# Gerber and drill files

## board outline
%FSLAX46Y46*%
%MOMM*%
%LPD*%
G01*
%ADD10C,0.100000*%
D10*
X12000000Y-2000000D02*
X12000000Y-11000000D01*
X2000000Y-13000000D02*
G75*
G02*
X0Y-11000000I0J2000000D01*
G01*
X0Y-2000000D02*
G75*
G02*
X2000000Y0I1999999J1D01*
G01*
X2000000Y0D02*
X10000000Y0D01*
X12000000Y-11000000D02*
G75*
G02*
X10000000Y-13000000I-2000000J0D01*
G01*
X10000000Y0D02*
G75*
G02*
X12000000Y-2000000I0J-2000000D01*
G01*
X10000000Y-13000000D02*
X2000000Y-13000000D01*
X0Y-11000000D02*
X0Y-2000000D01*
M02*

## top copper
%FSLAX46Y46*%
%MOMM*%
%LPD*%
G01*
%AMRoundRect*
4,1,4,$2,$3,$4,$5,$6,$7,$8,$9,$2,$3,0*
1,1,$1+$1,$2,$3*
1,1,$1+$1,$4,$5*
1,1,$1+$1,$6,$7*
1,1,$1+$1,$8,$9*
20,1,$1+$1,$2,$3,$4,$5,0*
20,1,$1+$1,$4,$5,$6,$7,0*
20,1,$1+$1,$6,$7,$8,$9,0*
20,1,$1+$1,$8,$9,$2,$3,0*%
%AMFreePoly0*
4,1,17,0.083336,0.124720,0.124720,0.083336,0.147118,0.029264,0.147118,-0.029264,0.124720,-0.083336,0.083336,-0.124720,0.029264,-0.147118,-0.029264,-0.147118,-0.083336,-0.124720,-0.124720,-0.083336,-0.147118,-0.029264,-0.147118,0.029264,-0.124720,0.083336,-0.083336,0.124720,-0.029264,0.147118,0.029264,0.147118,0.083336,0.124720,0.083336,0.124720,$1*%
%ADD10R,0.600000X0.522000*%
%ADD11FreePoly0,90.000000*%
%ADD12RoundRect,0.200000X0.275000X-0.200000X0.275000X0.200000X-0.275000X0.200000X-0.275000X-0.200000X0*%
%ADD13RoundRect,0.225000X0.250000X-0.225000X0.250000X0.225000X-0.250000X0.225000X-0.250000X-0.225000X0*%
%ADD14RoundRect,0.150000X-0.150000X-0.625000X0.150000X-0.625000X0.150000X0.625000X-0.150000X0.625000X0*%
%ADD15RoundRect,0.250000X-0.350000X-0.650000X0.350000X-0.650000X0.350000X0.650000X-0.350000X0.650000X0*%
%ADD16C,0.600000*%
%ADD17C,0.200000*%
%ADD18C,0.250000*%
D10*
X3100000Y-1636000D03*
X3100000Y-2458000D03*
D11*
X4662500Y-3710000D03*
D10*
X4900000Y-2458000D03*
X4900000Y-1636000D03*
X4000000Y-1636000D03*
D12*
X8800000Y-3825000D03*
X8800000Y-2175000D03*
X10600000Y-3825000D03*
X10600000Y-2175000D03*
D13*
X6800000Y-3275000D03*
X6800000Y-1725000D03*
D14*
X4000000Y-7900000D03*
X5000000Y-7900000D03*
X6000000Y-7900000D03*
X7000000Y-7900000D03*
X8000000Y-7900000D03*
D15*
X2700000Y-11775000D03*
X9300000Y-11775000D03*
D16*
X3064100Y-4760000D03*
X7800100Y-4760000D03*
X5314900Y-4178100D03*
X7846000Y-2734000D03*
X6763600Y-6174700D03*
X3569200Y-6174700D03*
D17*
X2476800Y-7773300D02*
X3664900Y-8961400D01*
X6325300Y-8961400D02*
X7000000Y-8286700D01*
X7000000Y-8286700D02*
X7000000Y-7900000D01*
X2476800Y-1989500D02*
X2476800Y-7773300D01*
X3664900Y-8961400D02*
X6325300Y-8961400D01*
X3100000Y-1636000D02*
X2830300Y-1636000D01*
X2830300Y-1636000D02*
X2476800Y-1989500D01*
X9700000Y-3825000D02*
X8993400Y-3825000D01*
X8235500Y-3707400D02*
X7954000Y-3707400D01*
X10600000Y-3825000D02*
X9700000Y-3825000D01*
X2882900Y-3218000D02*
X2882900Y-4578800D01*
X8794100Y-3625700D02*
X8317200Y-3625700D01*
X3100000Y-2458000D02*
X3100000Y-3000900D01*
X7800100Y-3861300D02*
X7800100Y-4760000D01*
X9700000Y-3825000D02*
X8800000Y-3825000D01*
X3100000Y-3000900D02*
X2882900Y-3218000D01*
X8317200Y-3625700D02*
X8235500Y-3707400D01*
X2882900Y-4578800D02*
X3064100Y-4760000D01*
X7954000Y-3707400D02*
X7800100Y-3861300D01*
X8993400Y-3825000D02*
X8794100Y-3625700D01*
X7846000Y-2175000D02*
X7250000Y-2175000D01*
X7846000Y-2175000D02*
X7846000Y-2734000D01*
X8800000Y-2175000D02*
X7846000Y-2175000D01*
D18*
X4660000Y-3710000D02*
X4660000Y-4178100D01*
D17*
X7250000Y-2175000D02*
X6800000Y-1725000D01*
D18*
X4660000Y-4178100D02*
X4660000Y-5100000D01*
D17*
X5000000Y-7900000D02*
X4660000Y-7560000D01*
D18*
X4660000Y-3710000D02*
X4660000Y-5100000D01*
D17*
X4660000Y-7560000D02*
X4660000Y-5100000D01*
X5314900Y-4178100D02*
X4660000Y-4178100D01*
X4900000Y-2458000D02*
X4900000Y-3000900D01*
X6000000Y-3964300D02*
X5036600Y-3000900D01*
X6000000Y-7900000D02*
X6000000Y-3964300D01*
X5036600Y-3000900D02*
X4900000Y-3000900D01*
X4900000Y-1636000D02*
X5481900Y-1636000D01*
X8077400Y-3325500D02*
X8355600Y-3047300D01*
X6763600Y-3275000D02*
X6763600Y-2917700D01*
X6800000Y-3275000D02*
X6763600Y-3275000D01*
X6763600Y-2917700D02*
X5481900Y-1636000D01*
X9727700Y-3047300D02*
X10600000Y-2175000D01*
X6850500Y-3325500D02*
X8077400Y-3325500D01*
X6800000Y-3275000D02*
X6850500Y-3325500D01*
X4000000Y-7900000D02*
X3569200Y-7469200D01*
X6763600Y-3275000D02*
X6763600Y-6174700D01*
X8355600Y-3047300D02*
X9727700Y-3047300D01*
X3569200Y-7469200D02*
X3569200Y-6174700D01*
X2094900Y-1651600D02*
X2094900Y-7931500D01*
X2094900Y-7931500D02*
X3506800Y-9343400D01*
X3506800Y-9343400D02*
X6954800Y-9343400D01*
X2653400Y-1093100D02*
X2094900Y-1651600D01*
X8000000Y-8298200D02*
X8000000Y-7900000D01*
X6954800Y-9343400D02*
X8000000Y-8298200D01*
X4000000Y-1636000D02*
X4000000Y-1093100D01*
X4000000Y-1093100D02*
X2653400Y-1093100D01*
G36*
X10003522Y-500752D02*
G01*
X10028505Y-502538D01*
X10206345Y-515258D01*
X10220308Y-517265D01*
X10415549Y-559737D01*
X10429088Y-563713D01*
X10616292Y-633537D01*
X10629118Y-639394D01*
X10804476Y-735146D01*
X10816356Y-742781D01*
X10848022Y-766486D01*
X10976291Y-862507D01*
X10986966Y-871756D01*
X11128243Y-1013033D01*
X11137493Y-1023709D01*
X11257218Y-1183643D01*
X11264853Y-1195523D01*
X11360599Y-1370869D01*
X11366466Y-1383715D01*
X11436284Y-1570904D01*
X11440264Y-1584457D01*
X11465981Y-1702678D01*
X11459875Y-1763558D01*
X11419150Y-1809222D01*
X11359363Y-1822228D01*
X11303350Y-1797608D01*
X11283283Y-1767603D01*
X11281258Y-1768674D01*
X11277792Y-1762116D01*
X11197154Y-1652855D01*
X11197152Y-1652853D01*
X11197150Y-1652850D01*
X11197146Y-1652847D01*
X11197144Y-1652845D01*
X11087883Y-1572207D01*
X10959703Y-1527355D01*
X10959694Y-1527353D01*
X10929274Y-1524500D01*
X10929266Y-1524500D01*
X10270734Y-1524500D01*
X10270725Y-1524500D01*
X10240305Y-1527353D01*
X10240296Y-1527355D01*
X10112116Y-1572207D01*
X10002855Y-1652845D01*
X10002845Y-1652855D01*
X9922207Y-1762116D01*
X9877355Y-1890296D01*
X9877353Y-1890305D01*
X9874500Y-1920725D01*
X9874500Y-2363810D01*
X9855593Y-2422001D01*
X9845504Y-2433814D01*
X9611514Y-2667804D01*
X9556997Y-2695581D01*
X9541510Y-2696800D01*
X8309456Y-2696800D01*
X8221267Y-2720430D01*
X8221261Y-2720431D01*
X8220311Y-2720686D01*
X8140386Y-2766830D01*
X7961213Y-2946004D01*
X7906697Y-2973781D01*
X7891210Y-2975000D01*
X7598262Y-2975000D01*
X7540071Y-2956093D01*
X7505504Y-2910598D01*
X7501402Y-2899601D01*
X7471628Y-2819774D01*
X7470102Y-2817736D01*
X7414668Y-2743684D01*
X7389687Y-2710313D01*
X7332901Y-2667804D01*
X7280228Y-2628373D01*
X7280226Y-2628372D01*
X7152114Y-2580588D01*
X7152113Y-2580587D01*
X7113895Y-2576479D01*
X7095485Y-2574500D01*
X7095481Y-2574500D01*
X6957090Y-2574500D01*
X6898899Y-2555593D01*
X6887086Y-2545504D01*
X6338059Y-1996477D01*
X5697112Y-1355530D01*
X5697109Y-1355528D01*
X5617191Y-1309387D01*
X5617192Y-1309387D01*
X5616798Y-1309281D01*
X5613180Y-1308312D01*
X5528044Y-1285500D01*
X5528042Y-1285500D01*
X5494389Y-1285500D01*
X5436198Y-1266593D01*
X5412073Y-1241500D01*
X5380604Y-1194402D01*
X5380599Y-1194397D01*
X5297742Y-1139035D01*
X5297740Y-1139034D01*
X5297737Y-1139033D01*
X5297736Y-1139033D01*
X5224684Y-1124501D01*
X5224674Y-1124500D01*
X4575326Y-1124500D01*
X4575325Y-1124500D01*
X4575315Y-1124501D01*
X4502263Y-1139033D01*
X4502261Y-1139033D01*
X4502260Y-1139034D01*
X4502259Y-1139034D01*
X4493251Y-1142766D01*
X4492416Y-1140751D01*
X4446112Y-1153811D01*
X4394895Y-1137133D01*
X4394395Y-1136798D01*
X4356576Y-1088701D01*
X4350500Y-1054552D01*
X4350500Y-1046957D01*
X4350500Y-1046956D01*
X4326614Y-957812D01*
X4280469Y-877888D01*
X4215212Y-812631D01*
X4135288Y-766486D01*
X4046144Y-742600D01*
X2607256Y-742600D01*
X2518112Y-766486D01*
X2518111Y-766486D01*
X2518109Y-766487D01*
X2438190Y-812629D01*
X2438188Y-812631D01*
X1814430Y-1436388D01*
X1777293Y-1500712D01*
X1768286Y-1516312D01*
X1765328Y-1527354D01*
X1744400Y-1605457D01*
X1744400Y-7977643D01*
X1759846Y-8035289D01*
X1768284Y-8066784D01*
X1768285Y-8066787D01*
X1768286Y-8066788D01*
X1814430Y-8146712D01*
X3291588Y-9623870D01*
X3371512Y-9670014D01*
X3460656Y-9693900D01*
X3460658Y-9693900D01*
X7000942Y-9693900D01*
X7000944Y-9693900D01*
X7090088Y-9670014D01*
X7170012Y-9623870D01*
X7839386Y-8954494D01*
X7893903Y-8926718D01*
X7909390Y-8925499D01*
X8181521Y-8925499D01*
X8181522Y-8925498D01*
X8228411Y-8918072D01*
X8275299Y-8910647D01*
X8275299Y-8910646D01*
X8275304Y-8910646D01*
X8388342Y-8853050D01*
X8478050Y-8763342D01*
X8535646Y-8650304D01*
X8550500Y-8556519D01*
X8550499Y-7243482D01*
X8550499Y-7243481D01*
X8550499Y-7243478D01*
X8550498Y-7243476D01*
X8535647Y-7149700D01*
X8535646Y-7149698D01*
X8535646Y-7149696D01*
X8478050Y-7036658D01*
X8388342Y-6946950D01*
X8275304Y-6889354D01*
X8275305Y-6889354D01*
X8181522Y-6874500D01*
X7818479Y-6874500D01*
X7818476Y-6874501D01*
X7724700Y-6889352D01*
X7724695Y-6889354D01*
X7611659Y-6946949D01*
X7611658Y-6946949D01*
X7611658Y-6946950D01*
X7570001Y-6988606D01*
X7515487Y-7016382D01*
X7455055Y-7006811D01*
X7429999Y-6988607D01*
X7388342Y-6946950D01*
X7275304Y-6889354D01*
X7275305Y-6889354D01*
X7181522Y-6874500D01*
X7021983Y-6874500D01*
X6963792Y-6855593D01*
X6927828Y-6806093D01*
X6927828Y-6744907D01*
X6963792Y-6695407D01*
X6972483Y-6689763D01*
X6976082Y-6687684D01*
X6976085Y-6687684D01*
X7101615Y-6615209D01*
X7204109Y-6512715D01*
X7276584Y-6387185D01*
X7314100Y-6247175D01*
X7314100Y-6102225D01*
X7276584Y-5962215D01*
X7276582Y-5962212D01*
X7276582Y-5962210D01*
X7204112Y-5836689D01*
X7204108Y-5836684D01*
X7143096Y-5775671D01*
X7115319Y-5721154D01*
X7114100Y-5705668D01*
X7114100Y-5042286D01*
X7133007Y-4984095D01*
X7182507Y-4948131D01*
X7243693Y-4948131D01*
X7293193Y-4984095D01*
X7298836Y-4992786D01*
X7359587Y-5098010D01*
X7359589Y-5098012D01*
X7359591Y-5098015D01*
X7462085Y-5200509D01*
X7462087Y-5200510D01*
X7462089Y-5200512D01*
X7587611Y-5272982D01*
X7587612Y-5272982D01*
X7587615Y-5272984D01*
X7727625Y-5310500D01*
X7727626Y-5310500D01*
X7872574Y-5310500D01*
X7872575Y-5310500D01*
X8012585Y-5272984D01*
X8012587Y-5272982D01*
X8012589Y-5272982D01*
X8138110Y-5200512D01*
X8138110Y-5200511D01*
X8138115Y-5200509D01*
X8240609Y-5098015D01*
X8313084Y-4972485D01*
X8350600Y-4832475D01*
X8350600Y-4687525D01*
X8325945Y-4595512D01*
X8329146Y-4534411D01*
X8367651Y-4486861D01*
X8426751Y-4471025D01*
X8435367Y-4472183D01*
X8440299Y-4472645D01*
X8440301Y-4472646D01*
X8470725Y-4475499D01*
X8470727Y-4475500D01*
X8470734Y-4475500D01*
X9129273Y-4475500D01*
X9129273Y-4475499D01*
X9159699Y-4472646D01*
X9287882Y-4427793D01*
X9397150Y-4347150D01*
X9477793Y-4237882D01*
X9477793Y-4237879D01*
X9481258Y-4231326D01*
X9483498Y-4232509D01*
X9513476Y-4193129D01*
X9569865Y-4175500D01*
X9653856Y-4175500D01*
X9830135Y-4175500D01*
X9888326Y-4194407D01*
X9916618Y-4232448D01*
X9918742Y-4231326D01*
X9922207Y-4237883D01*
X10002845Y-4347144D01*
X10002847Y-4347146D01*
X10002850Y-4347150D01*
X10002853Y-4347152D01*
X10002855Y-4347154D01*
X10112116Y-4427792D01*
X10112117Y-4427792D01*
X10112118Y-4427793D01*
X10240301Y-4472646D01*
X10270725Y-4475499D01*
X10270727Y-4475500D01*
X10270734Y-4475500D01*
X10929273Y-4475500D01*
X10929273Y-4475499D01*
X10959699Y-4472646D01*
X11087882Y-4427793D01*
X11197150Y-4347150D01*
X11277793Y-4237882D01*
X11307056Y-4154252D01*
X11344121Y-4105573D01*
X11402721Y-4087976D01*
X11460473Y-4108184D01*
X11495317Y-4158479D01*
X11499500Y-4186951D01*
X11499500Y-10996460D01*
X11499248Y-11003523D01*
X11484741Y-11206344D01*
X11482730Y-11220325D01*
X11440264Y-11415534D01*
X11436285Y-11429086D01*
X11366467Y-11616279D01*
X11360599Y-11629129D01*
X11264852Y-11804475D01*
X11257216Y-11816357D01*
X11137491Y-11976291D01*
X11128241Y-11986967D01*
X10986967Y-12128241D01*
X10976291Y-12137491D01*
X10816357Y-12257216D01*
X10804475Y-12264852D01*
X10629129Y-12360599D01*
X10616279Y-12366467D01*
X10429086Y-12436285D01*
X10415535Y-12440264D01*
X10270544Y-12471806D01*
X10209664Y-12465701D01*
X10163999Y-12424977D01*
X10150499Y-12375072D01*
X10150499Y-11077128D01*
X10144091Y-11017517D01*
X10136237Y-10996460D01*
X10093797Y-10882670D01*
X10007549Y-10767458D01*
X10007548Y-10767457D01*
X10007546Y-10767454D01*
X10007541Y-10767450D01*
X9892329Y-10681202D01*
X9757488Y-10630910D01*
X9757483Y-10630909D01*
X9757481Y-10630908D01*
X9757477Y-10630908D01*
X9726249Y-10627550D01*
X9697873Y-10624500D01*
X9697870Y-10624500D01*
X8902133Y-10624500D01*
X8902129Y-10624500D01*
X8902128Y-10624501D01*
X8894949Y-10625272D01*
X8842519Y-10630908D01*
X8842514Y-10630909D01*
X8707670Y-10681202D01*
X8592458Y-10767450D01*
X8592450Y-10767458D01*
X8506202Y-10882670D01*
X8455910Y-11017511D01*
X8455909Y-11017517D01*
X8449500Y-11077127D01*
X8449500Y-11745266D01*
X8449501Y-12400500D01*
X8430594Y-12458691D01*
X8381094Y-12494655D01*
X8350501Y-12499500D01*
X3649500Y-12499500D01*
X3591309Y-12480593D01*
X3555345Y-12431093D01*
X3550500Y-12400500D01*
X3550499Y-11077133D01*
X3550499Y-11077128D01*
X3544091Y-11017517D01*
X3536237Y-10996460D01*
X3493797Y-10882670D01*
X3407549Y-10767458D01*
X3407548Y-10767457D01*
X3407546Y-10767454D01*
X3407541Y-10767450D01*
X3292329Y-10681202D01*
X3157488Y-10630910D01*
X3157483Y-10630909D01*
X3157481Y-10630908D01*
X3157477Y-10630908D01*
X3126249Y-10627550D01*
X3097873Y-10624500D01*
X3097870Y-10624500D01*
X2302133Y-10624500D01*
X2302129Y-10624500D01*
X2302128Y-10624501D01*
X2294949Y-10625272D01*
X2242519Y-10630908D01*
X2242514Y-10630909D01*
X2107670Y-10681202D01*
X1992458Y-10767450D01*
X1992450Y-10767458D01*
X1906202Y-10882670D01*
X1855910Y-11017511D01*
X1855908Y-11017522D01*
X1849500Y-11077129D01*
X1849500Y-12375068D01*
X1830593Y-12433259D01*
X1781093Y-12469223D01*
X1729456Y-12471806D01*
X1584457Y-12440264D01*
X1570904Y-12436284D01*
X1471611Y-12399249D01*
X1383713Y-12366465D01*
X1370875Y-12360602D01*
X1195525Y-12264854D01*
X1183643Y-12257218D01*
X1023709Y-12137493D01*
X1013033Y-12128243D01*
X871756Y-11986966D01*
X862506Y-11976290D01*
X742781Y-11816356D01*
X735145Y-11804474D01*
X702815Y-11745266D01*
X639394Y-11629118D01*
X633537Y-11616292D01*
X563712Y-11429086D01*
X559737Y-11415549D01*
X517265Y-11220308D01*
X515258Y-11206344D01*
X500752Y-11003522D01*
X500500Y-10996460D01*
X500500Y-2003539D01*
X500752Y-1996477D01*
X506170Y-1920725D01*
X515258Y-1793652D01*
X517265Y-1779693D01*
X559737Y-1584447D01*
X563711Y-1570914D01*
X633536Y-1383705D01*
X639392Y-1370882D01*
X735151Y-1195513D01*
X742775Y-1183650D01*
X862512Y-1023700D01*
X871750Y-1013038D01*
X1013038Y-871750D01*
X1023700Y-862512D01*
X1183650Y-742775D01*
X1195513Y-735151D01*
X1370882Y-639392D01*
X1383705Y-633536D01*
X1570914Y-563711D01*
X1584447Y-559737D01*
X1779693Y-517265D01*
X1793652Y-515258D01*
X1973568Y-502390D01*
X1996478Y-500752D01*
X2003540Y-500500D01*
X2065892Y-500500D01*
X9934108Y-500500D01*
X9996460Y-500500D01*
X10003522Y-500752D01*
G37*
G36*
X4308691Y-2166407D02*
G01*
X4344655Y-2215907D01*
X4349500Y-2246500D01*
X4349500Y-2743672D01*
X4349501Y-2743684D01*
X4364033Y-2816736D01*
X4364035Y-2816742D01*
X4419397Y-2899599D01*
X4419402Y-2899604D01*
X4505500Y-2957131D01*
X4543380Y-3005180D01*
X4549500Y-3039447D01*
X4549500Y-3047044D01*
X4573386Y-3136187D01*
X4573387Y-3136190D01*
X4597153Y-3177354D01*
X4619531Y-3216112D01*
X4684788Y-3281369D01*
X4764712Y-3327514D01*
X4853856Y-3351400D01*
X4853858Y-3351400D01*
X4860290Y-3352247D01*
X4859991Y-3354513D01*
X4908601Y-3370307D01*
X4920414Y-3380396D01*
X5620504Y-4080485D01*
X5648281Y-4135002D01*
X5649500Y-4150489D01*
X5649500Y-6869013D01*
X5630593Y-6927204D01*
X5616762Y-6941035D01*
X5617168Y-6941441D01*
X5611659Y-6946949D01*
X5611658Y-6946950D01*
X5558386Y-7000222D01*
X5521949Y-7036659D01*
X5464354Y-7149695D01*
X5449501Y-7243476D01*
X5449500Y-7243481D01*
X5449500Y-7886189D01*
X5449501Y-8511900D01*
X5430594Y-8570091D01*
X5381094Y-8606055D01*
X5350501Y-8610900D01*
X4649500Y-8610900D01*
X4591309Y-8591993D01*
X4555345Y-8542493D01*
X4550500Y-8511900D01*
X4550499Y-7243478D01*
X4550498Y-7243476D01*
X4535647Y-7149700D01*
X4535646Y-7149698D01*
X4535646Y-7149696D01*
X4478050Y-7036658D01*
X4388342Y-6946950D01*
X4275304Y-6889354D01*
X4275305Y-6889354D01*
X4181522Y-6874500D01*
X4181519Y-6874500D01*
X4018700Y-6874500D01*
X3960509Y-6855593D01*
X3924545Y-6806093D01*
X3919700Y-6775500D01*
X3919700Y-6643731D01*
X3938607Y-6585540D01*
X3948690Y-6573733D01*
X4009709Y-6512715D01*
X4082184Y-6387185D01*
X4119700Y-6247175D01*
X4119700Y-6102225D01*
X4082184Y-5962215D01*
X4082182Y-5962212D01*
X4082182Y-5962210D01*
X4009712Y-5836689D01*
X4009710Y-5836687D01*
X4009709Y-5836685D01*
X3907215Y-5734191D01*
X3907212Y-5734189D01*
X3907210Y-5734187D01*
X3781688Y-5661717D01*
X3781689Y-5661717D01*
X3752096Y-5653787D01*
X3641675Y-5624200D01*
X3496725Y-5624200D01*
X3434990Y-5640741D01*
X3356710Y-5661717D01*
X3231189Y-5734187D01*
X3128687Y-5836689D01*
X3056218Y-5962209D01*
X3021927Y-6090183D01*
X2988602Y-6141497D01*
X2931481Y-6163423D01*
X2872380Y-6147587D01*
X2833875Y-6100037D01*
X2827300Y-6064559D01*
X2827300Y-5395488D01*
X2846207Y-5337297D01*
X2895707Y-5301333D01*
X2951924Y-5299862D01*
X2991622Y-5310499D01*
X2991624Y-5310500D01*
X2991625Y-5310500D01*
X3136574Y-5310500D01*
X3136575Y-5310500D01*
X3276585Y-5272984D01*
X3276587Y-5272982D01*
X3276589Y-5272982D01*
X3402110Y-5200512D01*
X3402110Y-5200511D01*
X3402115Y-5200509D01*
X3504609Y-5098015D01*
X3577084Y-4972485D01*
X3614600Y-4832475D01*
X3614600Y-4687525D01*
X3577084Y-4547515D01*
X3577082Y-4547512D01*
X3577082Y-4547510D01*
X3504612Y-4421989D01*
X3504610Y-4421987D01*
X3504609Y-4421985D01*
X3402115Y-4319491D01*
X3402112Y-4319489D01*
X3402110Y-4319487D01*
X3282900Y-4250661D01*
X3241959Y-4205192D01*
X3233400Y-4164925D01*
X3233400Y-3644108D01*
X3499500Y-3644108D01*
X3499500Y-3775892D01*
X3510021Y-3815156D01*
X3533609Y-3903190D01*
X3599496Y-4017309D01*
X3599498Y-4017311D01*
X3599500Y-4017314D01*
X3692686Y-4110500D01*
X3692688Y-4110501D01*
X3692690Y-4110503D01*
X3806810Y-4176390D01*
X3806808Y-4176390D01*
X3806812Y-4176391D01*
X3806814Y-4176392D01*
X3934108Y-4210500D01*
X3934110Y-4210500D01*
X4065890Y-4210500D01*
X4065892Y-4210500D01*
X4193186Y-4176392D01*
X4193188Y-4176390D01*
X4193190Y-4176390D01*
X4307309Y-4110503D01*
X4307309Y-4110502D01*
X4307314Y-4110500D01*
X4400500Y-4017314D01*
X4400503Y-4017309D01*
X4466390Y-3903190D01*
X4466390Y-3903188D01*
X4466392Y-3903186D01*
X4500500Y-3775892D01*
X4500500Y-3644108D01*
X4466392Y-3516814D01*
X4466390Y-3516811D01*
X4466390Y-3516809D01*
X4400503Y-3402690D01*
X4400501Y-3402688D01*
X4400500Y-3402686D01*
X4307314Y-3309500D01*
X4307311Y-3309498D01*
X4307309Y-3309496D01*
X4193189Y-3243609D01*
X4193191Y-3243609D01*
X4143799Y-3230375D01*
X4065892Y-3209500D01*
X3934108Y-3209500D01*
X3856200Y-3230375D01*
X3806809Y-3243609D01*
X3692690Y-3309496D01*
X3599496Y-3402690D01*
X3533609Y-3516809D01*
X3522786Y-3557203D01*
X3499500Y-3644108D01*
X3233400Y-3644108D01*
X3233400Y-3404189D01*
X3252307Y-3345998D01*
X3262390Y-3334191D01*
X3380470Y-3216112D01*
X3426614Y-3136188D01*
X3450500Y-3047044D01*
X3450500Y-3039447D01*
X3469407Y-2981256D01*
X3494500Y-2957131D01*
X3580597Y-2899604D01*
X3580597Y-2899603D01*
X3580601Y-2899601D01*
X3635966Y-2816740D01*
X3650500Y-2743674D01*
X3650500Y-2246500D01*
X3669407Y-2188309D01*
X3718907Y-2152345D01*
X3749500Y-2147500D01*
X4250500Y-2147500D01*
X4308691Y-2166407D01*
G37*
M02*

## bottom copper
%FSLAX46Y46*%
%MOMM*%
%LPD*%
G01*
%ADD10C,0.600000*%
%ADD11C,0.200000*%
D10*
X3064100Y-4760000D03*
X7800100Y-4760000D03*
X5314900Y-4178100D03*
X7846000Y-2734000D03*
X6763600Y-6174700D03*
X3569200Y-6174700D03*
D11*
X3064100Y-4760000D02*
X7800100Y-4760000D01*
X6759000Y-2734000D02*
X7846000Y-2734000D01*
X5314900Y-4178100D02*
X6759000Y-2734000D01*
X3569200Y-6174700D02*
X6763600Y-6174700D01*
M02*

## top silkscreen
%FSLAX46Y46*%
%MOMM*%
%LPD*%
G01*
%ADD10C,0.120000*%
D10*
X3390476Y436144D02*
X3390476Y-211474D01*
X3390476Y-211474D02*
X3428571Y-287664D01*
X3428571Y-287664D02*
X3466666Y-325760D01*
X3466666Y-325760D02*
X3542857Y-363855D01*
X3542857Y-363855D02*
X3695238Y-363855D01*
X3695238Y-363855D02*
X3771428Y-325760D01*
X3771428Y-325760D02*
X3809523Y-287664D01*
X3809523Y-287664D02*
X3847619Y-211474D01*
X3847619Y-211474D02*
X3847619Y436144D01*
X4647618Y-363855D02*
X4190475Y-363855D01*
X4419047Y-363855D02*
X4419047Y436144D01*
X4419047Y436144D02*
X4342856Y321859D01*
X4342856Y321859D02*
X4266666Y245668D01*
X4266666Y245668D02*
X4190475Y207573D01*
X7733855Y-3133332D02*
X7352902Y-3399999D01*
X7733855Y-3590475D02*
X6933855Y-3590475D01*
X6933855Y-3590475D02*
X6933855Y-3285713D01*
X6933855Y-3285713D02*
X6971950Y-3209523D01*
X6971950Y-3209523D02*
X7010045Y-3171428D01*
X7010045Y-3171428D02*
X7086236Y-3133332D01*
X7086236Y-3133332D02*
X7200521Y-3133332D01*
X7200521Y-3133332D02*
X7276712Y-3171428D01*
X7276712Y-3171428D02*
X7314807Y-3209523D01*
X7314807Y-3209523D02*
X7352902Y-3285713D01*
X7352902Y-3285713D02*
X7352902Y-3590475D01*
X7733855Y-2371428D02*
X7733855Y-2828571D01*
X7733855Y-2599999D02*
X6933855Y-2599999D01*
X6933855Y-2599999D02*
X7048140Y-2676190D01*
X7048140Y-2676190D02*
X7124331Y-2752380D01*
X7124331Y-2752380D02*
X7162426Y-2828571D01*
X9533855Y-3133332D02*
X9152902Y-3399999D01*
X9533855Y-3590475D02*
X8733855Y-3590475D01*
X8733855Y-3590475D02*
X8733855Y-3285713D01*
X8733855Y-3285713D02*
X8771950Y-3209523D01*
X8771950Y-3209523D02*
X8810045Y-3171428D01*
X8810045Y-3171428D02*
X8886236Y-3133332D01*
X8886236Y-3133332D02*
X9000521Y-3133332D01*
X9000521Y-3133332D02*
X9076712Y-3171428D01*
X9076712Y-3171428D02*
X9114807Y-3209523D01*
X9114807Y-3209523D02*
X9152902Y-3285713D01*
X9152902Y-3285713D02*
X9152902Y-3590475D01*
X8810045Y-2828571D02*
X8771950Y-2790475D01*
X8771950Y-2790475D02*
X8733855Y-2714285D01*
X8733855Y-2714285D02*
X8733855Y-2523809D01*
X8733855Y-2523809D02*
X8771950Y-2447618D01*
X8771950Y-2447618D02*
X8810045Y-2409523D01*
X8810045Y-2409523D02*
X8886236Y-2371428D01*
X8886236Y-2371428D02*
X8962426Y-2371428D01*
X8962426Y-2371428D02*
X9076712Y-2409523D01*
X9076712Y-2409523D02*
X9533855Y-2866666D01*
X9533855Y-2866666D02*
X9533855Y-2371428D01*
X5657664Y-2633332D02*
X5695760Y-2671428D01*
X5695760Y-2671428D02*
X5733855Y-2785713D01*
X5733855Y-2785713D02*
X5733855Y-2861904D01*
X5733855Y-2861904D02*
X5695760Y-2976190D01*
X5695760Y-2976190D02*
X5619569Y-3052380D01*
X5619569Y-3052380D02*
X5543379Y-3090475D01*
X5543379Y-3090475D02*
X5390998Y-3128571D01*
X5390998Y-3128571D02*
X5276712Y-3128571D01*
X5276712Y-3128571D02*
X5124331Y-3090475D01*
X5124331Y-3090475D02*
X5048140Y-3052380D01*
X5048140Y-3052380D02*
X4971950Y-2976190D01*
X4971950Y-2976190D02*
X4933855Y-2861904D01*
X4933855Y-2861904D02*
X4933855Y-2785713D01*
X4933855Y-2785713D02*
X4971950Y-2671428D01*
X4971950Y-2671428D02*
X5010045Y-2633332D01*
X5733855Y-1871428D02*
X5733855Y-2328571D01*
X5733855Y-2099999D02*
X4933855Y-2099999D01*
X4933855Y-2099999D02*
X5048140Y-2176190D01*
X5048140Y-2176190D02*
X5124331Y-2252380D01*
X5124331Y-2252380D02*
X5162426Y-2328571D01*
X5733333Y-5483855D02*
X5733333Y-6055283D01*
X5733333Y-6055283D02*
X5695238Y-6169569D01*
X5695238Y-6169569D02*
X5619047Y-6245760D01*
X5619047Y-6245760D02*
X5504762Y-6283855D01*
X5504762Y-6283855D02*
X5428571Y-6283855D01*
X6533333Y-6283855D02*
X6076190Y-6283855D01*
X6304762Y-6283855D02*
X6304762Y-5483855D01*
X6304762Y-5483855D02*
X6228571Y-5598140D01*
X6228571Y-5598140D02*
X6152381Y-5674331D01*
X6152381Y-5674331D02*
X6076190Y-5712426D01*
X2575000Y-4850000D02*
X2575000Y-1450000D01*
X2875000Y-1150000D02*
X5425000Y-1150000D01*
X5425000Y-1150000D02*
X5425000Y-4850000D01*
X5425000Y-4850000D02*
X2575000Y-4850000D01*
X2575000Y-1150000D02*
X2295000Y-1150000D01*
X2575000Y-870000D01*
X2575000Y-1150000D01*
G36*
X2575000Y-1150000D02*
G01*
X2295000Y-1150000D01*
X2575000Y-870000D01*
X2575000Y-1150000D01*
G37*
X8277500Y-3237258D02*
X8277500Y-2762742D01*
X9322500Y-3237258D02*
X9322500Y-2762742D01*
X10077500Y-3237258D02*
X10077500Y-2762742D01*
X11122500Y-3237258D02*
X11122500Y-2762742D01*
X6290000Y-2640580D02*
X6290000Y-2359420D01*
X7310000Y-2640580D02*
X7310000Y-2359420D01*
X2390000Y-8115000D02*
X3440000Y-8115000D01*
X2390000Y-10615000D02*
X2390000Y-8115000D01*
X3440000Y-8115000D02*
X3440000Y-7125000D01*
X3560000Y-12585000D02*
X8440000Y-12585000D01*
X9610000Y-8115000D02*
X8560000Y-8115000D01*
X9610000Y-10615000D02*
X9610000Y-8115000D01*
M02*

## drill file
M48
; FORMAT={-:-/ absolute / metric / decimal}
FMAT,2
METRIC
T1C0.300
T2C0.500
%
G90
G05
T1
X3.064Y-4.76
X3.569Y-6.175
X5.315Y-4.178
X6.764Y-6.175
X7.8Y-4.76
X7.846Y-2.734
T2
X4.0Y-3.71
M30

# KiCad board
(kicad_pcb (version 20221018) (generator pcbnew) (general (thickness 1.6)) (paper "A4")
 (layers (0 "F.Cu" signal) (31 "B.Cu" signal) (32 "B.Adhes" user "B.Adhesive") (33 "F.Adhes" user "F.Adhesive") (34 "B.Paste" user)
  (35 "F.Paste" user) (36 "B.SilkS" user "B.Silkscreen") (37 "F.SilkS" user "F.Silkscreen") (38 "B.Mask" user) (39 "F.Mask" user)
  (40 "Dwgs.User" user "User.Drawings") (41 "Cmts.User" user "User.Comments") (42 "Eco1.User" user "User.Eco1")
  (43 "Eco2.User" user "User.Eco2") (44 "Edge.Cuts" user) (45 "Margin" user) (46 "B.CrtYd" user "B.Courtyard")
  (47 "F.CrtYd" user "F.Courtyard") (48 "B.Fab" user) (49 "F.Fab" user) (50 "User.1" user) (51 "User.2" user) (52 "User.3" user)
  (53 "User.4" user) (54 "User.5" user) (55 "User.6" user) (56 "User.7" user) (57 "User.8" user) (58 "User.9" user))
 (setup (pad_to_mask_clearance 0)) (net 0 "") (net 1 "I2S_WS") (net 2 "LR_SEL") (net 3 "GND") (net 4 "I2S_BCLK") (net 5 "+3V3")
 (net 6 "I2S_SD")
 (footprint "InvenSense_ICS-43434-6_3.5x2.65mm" (layer "F.Cu") (at 4 3)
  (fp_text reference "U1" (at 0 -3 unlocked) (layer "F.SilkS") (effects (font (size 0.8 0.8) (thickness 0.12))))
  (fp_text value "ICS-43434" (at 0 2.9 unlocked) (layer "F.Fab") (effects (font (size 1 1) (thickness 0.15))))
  (fp_line (start -1.425 1.85) (end -1.425 -1.55) (stroke (width 0.12) (type default)) (layer "F.SilkS"))
  (fp_line (start -1.125 -1.85) (end 1.425 -1.85) (stroke (width 0.12) (type default)) (layer "F.SilkS"))
  (fp_line (start 1.425 -1.85) (end 1.425 1.85) (stroke (width 0.12) (type default)) (layer "F.SilkS"))
  (fp_line (start 1.425 1.85) (end -1.425 1.85) (stroke (width 0.12) (type default)) (layer "F.SilkS"))
  (fp_poly
   (pts (xy -1.425 -1.85) (xy -1.705 -1.85) (xy -1.425 -2.13) (xy -1.425 -1.85)) (stroke (width 0.12) (type solid)) (fill solid)
   (layer "F.SilkS"))
  (pad "" np_thru_hole circle (at 0 0.71) (size 0.5 0.5) (drill 0.5) (layers "*.Mask"))
  (pad "1" smd rect (at -0.9 -1.364) (size 0.6 0.522) (layers "F.Cu" "F.Mask") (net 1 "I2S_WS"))
  (pad "2" smd rect (at -0.9 -0.542) (size 0.6 0.522) (layers "F.Cu" "F.Mask") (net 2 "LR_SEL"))
  (pad "3" smd custom (at 0.6625 0.71 90) (size 0.3 0.3) (layers "F.Cu" "F.Mask") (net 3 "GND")
   (options (clearance outline) (anchor circle)) (primitives))
  (pad "4" smd rect (at 0.9 -0.542) (size 0.6 0.522) (layers "F.Cu" "F.Mask") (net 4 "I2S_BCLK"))
  (pad "5" smd rect (at 0.9 -1.364) (size 0.6 0.522) (layers "F.Cu" "F.Mask") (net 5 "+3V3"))
  (pad "6" smd rect (at 0 -1.364) (size 0.6 0.522) (layers "F.Cu" "F.Mask") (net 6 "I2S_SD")))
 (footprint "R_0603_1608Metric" (layer "F.Cu") (at 8.8 3 90)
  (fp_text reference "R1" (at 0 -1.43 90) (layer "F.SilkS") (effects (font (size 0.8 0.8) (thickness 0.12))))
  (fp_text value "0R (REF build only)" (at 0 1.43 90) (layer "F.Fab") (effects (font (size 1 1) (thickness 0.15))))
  (fp_line (start -0.237258 -0.5225) (end 0.237258 -0.5225) (stroke (width 0.12) (type solid)) (layer "F.SilkS"))
  (fp_line (start -0.237258 0.5225) (end 0.237258 0.5225) (stroke (width 0.12) (type solid)) (layer "F.SilkS"))
  (pad "1" smd roundrect (at -0.825 0 90) (size 0.8 0.95) (layers "F.Cu" "F.Paste" "F.Mask") (roundrect_rratio 0.25) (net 2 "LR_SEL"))
  (pad "2" smd roundrect (at 0.825 0 90) (size 0.8 0.95) (layers "F.Cu" "F.Paste" "F.Mask") (roundrect_rratio 0.25) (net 3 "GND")))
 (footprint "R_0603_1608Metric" (layer "F.Cu") (at 10.6 3 90)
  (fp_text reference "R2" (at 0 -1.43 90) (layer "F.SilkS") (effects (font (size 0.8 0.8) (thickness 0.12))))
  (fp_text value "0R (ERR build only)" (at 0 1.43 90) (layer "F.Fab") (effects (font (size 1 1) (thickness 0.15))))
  (fp_line (start -0.237258 -0.5225) (end 0.237258 -0.5225) (stroke (width 0.12) (type solid)) (layer "F.SilkS"))
  (fp_line (start -0.237258 0.5225) (end 0.237258 0.5225) (stroke (width 0.12) (type solid)) (layer "F.SilkS"))
  (pad "1" smd roundrect (at -0.825 0 90) (size 0.8 0.95) (layers "F.Cu" "F.Paste" "F.Mask") (roundrect_rratio 0.25) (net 2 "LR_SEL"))
  (pad "2" smd roundrect (at 0.825 0 90) (size 0.8 0.95) (layers "F.Cu" "F.Paste" "F.Mask") (roundrect_rratio 0.25) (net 5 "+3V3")))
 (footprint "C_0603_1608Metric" (layer "F.Cu") (at 6.8 2.5 90)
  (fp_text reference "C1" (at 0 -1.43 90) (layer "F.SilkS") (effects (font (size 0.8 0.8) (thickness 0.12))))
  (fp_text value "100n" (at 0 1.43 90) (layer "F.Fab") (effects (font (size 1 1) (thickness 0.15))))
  (fp_line (start -0.14058 -0.51) (end 0.14058 -0.51) (stroke (width 0.12) (type solid)) (layer "F.SilkS"))
  (fp_line (start -0.14058 0.51) (end 0.14058 0.51) (stroke (width 0.12) (type solid)) (layer "F.SilkS"))
  (pad "1" smd roundrect (at -0.775 0 90) (size 0.9 0.95) (layers "F.Cu" "F.Paste" "F.Mask") (roundrect_rratio 0.25) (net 5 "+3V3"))
  (pad "2" smd roundrect (at 0.775 0 90) (size 0.9 0.95) (layers "F.Cu" "F.Paste" "F.Mask") (roundrect_rratio 0.25) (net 3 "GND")))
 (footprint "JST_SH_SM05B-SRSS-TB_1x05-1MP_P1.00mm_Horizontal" (layer "F.Cu") (at 6 9.9)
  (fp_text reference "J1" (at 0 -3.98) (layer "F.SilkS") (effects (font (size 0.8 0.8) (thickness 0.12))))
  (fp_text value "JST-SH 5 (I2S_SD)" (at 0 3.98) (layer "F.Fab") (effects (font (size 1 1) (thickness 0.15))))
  (fp_line (start -3.61 -1.785) (end -2.56 -1.785) (stroke (width 0.12) (type solid)) (layer "F.SilkS"))
  (fp_line (start -3.61 0.715) (end -3.61 -1.785) (stroke (width 0.12) (type solid)) (layer "F.SilkS"))
  (fp_line (start -2.56 -1.785) (end -2.56 -2.775) (stroke (width 0.12) (type solid)) (layer "F.SilkS"))
  (fp_line (start -2.44 2.685) (end 2.44 2.685) (stroke (width 0.12) (type solid)) (layer "F.SilkS"))
  (fp_line (start 3.61 -1.785) (end 2.56 -1.785) (stroke (width 0.12) (type solid)) (layer "F.SilkS"))
  (fp_line (start 3.61 0.715) (end 3.61 -1.785) (stroke (width 0.12) (type solid)) (layer "F.SilkS"))
  (pad "1" smd roundrect (at -2 -2) (size 0.6 1.55) (layers "F.Cu" "F.Paste" "F.Mask") (roundrect_rratio 0.25) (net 5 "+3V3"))
  (pad "2" smd roundrect (at -1 -2) (size 0.6 1.55) (layers "F.Cu" "F.Paste" "F.Mask") (roundrect_rratio 0.25) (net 3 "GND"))
  (pad "3" smd roundrect (at 0 -2) (size 0.6 1.55) (layers "F.Cu" "F.Paste" "F.Mask") (roundrect_rratio 0.25) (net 4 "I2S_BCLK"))
  (pad "4" smd roundrect (at 1 -2) (size 0.6 1.55) (layers "F.Cu" "F.Paste" "F.Mask") (roundrect_rratio 0.25) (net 1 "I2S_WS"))
  (pad "5" smd roundrect (at 2 -2) (size 0.6 1.55) (layers "F.Cu" "F.Paste" "F.Mask") (roundrect_rratio 0.25) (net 6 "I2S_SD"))
  (pad "MP" smd roundrect (at -3.3 1.875) (size 1.2 1.8) (layers "F.Cu" "F.Paste" "F.Mask") (roundrect_rratio 0.208333))
  (pad "MP" smd roundrect (at 3.3 1.875) (size 1.2 1.8) (layers "F.Cu" "F.Paste" "F.Mask") (roundrect_rratio 0.208333)))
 (gr_line (start 12 2) (end 12 11) (stroke (width 0.1) (type default)) (layer "Edge.Cuts"))
 (gr_arc (start 2 13) (mid 0.585786 12.414213) (end 0 11) (stroke (width 0.1) (type default)) (layer "Edge.Cuts"))
 (gr_arc (start 0 2) (mid 0.585786 0.585786) (end 2 0) (stroke (width 0.1) (type default)) (layer "Edge.Cuts"))
 (gr_line (start 2 0) (end 10 0) (stroke (width 0.1) (type default)) (layer "Edge.Cuts"))
 (gr_arc (start 12 11) (mid 11.414213 12.414213) (end 10 13) (stroke (width 0.1) (type default)) (layer "Edge.Cuts"))
 (gr_arc (start 10 0) (mid 11.414213 0.585786) (end 12 2) (stroke (width 0.1) (type default)) (layer "Edge.Cuts"))
 (gr_line (start 10 13) (end 2 13) (stroke (width 0.1) (type default)) (layer "Edge.Cuts"))
 (gr_line (start 0 11) (end 0 2) (stroke (width 0.1) (type default)) (layer "Edge.Cuts"))
 (segment (start 2.4768 7.7733) (end 3.6649 8.9614) (width 0.2) (layer "F.Cu") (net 1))
 (segment (start 6.3253 8.9614) (end 7 8.2867) (width 0.2) (layer "F.Cu") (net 1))
 (segment (start 7 8.2867) (end 7 7.9) (width 0.2) (layer "F.Cu") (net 1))
 (segment (start 2.4768 1.9895) (end 2.4768 7.7733) (width 0.2) (layer "F.Cu") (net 1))
 (segment (start 3.6649 8.9614) (end 6.3253 8.9614) (width 0.2) (layer "F.Cu") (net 1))
 (segment (start 3.1 1.636) (end 2.8303 1.636) (width 0.2) (layer "F.Cu") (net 1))
 (segment (start 2.8303 1.636) (end 2.4768 1.9895) (width 0.2) (layer "F.Cu") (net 1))
 (segment (start 9.7 3.825) (end 8.9934 3.825) (width 0.2) (layer "F.Cu") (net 2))
 (segment (start 8.2355 3.7074) (end 7.954 3.7074) (width 0.2) (layer "F.Cu") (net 2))
 (segment (start 10.6 3.825) (end 9.7 3.825) (width 0.2) (layer "F.Cu") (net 2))
 (segment (start 2.8829 3.218) (end 2.8829 4.5788) (width 0.2) (layer "F.Cu") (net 2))
 (segment (start 8.7941 3.6257) (end 8.3172 3.6257) (width 0.2) (layer "F.Cu") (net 2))
 (segment (start 3.1 2.458) (end 3.1 3.0009) (width 0.2) (layer "F.Cu") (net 2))
 (segment (start 7.8001 3.8613) (end 7.8001 4.76) (width 0.2) (layer "F.Cu") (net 2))
 (segment (start 9.7 3.825) (end 8.8 3.825) (width 0.2) (layer "F.Cu") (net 2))
 (segment (start 3.1 3.0009) (end 2.8829 3.218) (width 0.2) (layer "F.Cu") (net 2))
 (segment (start 8.3172 3.6257) (end 8.2355 3.7074) (width 0.2) (layer "F.Cu") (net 2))
 (segment (start 2.8829 4.5788) (end 3.0641 4.76) (width 0.2) (layer "F.Cu") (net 2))
 (segment (start 7.954 3.7074) (end 7.8001 3.8613) (width 0.2) (layer "F.Cu") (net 2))
 (segment (start 8.9934 3.825) (end 8.7941 3.6257) (width 0.2) (layer "F.Cu") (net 2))
 (via (at 3.0641 4.76) (size 0.6) (drill 0.3) (layers "F.Cu" "B.Cu") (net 2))
 (via (at 7.8001 4.76) (size 0.6) (drill 0.3) (layers "F.Cu" "B.Cu") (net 2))
 (segment (start 3.0641 4.76) (end 7.8001 4.76) (width 0.2) (layer "B.Cu") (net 2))
 (segment (start 7.846 2.175) (end 7.25 2.175) (width 0.2) (layer "F.Cu") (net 3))
 (segment (start 7.846 2.175) (end 7.846 2.734) (width 0.2) (layer "F.Cu") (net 3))
 (segment (start 8.8 2.175) (end 7.846 2.175) (width 0.2) (layer "F.Cu") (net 3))
 (segment (start 4.66 3.71) (end 4.66 4.1781) (width 0.25) (layer "F.Cu") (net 3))
 (segment (start 7.25 2.175) (end 6.8 1.725) (width 0.2) (layer "F.Cu") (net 3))
 (segment (start 4.66 4.1781) (end 4.66 5.1) (width 0.25) (layer "F.Cu") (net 3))
 (segment (start 5 7.9) (end 4.66 7.56) (width 0.2) (layer "F.Cu") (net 3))
 (segment (start 4.66 3.71) (end 4.66 5.1) (width 0.25) (layer "F.Cu") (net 3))
 (segment (start 4.66 7.56) (end 4.66 5.1) (width 0.2) (layer "F.Cu") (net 3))
 (segment (start 5.3149 4.1781) (end 4.66 4.1781) (width 0.2) (layer "F.Cu") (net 3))
 (via (at 5.3149 4.1781) (size 0.6) (drill 0.3) (layers "F.Cu" "B.Cu") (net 3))
 (via (at 7.846 2.734) (size 0.6) (drill 0.3) (layers "F.Cu" "B.Cu") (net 3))
 (segment (start 6.759 2.734) (end 7.846 2.734) (width 0.2) (layer "B.Cu") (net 3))
 (segment (start 5.3149 4.1781) (end 6.759 2.734) (width 0.2) (layer "B.Cu") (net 3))
 (segment (start 4.9 2.458) (end 4.9 3.0009) (width 0.2) (layer "F.Cu") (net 4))
 (segment (start 6 3.9643) (end 5.0366 3.0009) (width 0.2) (layer "F.Cu") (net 4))
 (segment (start 6 7.9) (end 6 3.9643) (width 0.2) (layer "F.Cu") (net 4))
 (segment (start 5.0366 3.0009) (end 4.9 3.0009) (width 0.2) (layer "F.Cu") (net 4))
 (segment (start 4.9 1.636) (end 5.4819 1.636) (width 0.2) (layer "F.Cu") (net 5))
 (segment (start 8.0774 3.3255) (end 8.3556 3.0473) (width 0.2) (layer "F.Cu") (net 5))
 (segment (start 6.7636 3.275) (end 6.7636 2.9177) (width 0.2) (layer "F.Cu") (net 5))
 (segment (start 6.8 3.275) (end 6.7636 3.275) (width 0.2) (layer "F.Cu") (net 5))
 (segment (start 6.7636 2.9177) (end 5.4819 1.636) (width 0.2) (layer "F.Cu") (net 5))
 (segment (start 9.7277 3.0473) (end 10.6 2.175) (width 0.2) (layer "F.Cu") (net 5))
 (segment (start 6.8505 3.3255) (end 8.0774 3.3255) (width 0.2) (layer "F.Cu") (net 5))
 (segment (start 6.8 3.275) (end 6.8505 3.3255) (width 0.2) (layer "F.Cu") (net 5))
 (segment (start 4 7.9) (end 3.5692 7.4692) (width 0.2) (layer "F.Cu") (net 5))
 (segment (start 6.7636 3.275) (end 6.7636 6.1747) (width 0.2) (layer "F.Cu") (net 5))
 (segment (start 8.3556 3.0473) (end 9.7277 3.0473) (width 0.2) (layer "F.Cu") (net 5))
 (segment (start 3.5692 7.4692) (end 3.5692 6.1747) (width 0.2) (layer "F.Cu") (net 5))
 (via (at 6.7636 6.1747) (size 0.6) (drill 0.3) (layers "F.Cu" "B.Cu") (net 5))
 (via (at 3.5692 6.1747) (size 0.6) (drill 0.3) (layers "F.Cu" "B.Cu") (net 5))
 (segment (start 3.5692 6.1747) (end 6.7636 6.1747) (width 0.2) (layer "B.Cu") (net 5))
 (segment (start 2.0949 1.6516) (end 2.0949 7.9315) (width 0.2) (layer "F.Cu") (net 6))
 (segment (start 2.0949 7.9315) (end 3.5068 9.3434) (width 0.2) (layer "F.Cu") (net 6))
 (segment (start 3.5068 9.3434) (end 6.9548 9.3434) (width 0.2) (layer "F.Cu") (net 6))
 (segment (start 2.6534 1.0931) (end 2.0949 1.6516) (width 0.2) (layer "F.Cu") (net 6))
 (segment (start 8 8.2982) (end 8 7.9) (width 0.2) (layer "F.Cu") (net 6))
 (segment (start 6.9548 9.3434) (end 8 8.2982) (width 0.2) (layer "F.Cu") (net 6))
 (segment (start 4 1.636) (end 4 1.0931) (width 0.2) (layer "F.Cu") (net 6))
 (segment (start 4 1.0931) (end 2.6534 1.0931) (width 0.2) (layer "F.Cu") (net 6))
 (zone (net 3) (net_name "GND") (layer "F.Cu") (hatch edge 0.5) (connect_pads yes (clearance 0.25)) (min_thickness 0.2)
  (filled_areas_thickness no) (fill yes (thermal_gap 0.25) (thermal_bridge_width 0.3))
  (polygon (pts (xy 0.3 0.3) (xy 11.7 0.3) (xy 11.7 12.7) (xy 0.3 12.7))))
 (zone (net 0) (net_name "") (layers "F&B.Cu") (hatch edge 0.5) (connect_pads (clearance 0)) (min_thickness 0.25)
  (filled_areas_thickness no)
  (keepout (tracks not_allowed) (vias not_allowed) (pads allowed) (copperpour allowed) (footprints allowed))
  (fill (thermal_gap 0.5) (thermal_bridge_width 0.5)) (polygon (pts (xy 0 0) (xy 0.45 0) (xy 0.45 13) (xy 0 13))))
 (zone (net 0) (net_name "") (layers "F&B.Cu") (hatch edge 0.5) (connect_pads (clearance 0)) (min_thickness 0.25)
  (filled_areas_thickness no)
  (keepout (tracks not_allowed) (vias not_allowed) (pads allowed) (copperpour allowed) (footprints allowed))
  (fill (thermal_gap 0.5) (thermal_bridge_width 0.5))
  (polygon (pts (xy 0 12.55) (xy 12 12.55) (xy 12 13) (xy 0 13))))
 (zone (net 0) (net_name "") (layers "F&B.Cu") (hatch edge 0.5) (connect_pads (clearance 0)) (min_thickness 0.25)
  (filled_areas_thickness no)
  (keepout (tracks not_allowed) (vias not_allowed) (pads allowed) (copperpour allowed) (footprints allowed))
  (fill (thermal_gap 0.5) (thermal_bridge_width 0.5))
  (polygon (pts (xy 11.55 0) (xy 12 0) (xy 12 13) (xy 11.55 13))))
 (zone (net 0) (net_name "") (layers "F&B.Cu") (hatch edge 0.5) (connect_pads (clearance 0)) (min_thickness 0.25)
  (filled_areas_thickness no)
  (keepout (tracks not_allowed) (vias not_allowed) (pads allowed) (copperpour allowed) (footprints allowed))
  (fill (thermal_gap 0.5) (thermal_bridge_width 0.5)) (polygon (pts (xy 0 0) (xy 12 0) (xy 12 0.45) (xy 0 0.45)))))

